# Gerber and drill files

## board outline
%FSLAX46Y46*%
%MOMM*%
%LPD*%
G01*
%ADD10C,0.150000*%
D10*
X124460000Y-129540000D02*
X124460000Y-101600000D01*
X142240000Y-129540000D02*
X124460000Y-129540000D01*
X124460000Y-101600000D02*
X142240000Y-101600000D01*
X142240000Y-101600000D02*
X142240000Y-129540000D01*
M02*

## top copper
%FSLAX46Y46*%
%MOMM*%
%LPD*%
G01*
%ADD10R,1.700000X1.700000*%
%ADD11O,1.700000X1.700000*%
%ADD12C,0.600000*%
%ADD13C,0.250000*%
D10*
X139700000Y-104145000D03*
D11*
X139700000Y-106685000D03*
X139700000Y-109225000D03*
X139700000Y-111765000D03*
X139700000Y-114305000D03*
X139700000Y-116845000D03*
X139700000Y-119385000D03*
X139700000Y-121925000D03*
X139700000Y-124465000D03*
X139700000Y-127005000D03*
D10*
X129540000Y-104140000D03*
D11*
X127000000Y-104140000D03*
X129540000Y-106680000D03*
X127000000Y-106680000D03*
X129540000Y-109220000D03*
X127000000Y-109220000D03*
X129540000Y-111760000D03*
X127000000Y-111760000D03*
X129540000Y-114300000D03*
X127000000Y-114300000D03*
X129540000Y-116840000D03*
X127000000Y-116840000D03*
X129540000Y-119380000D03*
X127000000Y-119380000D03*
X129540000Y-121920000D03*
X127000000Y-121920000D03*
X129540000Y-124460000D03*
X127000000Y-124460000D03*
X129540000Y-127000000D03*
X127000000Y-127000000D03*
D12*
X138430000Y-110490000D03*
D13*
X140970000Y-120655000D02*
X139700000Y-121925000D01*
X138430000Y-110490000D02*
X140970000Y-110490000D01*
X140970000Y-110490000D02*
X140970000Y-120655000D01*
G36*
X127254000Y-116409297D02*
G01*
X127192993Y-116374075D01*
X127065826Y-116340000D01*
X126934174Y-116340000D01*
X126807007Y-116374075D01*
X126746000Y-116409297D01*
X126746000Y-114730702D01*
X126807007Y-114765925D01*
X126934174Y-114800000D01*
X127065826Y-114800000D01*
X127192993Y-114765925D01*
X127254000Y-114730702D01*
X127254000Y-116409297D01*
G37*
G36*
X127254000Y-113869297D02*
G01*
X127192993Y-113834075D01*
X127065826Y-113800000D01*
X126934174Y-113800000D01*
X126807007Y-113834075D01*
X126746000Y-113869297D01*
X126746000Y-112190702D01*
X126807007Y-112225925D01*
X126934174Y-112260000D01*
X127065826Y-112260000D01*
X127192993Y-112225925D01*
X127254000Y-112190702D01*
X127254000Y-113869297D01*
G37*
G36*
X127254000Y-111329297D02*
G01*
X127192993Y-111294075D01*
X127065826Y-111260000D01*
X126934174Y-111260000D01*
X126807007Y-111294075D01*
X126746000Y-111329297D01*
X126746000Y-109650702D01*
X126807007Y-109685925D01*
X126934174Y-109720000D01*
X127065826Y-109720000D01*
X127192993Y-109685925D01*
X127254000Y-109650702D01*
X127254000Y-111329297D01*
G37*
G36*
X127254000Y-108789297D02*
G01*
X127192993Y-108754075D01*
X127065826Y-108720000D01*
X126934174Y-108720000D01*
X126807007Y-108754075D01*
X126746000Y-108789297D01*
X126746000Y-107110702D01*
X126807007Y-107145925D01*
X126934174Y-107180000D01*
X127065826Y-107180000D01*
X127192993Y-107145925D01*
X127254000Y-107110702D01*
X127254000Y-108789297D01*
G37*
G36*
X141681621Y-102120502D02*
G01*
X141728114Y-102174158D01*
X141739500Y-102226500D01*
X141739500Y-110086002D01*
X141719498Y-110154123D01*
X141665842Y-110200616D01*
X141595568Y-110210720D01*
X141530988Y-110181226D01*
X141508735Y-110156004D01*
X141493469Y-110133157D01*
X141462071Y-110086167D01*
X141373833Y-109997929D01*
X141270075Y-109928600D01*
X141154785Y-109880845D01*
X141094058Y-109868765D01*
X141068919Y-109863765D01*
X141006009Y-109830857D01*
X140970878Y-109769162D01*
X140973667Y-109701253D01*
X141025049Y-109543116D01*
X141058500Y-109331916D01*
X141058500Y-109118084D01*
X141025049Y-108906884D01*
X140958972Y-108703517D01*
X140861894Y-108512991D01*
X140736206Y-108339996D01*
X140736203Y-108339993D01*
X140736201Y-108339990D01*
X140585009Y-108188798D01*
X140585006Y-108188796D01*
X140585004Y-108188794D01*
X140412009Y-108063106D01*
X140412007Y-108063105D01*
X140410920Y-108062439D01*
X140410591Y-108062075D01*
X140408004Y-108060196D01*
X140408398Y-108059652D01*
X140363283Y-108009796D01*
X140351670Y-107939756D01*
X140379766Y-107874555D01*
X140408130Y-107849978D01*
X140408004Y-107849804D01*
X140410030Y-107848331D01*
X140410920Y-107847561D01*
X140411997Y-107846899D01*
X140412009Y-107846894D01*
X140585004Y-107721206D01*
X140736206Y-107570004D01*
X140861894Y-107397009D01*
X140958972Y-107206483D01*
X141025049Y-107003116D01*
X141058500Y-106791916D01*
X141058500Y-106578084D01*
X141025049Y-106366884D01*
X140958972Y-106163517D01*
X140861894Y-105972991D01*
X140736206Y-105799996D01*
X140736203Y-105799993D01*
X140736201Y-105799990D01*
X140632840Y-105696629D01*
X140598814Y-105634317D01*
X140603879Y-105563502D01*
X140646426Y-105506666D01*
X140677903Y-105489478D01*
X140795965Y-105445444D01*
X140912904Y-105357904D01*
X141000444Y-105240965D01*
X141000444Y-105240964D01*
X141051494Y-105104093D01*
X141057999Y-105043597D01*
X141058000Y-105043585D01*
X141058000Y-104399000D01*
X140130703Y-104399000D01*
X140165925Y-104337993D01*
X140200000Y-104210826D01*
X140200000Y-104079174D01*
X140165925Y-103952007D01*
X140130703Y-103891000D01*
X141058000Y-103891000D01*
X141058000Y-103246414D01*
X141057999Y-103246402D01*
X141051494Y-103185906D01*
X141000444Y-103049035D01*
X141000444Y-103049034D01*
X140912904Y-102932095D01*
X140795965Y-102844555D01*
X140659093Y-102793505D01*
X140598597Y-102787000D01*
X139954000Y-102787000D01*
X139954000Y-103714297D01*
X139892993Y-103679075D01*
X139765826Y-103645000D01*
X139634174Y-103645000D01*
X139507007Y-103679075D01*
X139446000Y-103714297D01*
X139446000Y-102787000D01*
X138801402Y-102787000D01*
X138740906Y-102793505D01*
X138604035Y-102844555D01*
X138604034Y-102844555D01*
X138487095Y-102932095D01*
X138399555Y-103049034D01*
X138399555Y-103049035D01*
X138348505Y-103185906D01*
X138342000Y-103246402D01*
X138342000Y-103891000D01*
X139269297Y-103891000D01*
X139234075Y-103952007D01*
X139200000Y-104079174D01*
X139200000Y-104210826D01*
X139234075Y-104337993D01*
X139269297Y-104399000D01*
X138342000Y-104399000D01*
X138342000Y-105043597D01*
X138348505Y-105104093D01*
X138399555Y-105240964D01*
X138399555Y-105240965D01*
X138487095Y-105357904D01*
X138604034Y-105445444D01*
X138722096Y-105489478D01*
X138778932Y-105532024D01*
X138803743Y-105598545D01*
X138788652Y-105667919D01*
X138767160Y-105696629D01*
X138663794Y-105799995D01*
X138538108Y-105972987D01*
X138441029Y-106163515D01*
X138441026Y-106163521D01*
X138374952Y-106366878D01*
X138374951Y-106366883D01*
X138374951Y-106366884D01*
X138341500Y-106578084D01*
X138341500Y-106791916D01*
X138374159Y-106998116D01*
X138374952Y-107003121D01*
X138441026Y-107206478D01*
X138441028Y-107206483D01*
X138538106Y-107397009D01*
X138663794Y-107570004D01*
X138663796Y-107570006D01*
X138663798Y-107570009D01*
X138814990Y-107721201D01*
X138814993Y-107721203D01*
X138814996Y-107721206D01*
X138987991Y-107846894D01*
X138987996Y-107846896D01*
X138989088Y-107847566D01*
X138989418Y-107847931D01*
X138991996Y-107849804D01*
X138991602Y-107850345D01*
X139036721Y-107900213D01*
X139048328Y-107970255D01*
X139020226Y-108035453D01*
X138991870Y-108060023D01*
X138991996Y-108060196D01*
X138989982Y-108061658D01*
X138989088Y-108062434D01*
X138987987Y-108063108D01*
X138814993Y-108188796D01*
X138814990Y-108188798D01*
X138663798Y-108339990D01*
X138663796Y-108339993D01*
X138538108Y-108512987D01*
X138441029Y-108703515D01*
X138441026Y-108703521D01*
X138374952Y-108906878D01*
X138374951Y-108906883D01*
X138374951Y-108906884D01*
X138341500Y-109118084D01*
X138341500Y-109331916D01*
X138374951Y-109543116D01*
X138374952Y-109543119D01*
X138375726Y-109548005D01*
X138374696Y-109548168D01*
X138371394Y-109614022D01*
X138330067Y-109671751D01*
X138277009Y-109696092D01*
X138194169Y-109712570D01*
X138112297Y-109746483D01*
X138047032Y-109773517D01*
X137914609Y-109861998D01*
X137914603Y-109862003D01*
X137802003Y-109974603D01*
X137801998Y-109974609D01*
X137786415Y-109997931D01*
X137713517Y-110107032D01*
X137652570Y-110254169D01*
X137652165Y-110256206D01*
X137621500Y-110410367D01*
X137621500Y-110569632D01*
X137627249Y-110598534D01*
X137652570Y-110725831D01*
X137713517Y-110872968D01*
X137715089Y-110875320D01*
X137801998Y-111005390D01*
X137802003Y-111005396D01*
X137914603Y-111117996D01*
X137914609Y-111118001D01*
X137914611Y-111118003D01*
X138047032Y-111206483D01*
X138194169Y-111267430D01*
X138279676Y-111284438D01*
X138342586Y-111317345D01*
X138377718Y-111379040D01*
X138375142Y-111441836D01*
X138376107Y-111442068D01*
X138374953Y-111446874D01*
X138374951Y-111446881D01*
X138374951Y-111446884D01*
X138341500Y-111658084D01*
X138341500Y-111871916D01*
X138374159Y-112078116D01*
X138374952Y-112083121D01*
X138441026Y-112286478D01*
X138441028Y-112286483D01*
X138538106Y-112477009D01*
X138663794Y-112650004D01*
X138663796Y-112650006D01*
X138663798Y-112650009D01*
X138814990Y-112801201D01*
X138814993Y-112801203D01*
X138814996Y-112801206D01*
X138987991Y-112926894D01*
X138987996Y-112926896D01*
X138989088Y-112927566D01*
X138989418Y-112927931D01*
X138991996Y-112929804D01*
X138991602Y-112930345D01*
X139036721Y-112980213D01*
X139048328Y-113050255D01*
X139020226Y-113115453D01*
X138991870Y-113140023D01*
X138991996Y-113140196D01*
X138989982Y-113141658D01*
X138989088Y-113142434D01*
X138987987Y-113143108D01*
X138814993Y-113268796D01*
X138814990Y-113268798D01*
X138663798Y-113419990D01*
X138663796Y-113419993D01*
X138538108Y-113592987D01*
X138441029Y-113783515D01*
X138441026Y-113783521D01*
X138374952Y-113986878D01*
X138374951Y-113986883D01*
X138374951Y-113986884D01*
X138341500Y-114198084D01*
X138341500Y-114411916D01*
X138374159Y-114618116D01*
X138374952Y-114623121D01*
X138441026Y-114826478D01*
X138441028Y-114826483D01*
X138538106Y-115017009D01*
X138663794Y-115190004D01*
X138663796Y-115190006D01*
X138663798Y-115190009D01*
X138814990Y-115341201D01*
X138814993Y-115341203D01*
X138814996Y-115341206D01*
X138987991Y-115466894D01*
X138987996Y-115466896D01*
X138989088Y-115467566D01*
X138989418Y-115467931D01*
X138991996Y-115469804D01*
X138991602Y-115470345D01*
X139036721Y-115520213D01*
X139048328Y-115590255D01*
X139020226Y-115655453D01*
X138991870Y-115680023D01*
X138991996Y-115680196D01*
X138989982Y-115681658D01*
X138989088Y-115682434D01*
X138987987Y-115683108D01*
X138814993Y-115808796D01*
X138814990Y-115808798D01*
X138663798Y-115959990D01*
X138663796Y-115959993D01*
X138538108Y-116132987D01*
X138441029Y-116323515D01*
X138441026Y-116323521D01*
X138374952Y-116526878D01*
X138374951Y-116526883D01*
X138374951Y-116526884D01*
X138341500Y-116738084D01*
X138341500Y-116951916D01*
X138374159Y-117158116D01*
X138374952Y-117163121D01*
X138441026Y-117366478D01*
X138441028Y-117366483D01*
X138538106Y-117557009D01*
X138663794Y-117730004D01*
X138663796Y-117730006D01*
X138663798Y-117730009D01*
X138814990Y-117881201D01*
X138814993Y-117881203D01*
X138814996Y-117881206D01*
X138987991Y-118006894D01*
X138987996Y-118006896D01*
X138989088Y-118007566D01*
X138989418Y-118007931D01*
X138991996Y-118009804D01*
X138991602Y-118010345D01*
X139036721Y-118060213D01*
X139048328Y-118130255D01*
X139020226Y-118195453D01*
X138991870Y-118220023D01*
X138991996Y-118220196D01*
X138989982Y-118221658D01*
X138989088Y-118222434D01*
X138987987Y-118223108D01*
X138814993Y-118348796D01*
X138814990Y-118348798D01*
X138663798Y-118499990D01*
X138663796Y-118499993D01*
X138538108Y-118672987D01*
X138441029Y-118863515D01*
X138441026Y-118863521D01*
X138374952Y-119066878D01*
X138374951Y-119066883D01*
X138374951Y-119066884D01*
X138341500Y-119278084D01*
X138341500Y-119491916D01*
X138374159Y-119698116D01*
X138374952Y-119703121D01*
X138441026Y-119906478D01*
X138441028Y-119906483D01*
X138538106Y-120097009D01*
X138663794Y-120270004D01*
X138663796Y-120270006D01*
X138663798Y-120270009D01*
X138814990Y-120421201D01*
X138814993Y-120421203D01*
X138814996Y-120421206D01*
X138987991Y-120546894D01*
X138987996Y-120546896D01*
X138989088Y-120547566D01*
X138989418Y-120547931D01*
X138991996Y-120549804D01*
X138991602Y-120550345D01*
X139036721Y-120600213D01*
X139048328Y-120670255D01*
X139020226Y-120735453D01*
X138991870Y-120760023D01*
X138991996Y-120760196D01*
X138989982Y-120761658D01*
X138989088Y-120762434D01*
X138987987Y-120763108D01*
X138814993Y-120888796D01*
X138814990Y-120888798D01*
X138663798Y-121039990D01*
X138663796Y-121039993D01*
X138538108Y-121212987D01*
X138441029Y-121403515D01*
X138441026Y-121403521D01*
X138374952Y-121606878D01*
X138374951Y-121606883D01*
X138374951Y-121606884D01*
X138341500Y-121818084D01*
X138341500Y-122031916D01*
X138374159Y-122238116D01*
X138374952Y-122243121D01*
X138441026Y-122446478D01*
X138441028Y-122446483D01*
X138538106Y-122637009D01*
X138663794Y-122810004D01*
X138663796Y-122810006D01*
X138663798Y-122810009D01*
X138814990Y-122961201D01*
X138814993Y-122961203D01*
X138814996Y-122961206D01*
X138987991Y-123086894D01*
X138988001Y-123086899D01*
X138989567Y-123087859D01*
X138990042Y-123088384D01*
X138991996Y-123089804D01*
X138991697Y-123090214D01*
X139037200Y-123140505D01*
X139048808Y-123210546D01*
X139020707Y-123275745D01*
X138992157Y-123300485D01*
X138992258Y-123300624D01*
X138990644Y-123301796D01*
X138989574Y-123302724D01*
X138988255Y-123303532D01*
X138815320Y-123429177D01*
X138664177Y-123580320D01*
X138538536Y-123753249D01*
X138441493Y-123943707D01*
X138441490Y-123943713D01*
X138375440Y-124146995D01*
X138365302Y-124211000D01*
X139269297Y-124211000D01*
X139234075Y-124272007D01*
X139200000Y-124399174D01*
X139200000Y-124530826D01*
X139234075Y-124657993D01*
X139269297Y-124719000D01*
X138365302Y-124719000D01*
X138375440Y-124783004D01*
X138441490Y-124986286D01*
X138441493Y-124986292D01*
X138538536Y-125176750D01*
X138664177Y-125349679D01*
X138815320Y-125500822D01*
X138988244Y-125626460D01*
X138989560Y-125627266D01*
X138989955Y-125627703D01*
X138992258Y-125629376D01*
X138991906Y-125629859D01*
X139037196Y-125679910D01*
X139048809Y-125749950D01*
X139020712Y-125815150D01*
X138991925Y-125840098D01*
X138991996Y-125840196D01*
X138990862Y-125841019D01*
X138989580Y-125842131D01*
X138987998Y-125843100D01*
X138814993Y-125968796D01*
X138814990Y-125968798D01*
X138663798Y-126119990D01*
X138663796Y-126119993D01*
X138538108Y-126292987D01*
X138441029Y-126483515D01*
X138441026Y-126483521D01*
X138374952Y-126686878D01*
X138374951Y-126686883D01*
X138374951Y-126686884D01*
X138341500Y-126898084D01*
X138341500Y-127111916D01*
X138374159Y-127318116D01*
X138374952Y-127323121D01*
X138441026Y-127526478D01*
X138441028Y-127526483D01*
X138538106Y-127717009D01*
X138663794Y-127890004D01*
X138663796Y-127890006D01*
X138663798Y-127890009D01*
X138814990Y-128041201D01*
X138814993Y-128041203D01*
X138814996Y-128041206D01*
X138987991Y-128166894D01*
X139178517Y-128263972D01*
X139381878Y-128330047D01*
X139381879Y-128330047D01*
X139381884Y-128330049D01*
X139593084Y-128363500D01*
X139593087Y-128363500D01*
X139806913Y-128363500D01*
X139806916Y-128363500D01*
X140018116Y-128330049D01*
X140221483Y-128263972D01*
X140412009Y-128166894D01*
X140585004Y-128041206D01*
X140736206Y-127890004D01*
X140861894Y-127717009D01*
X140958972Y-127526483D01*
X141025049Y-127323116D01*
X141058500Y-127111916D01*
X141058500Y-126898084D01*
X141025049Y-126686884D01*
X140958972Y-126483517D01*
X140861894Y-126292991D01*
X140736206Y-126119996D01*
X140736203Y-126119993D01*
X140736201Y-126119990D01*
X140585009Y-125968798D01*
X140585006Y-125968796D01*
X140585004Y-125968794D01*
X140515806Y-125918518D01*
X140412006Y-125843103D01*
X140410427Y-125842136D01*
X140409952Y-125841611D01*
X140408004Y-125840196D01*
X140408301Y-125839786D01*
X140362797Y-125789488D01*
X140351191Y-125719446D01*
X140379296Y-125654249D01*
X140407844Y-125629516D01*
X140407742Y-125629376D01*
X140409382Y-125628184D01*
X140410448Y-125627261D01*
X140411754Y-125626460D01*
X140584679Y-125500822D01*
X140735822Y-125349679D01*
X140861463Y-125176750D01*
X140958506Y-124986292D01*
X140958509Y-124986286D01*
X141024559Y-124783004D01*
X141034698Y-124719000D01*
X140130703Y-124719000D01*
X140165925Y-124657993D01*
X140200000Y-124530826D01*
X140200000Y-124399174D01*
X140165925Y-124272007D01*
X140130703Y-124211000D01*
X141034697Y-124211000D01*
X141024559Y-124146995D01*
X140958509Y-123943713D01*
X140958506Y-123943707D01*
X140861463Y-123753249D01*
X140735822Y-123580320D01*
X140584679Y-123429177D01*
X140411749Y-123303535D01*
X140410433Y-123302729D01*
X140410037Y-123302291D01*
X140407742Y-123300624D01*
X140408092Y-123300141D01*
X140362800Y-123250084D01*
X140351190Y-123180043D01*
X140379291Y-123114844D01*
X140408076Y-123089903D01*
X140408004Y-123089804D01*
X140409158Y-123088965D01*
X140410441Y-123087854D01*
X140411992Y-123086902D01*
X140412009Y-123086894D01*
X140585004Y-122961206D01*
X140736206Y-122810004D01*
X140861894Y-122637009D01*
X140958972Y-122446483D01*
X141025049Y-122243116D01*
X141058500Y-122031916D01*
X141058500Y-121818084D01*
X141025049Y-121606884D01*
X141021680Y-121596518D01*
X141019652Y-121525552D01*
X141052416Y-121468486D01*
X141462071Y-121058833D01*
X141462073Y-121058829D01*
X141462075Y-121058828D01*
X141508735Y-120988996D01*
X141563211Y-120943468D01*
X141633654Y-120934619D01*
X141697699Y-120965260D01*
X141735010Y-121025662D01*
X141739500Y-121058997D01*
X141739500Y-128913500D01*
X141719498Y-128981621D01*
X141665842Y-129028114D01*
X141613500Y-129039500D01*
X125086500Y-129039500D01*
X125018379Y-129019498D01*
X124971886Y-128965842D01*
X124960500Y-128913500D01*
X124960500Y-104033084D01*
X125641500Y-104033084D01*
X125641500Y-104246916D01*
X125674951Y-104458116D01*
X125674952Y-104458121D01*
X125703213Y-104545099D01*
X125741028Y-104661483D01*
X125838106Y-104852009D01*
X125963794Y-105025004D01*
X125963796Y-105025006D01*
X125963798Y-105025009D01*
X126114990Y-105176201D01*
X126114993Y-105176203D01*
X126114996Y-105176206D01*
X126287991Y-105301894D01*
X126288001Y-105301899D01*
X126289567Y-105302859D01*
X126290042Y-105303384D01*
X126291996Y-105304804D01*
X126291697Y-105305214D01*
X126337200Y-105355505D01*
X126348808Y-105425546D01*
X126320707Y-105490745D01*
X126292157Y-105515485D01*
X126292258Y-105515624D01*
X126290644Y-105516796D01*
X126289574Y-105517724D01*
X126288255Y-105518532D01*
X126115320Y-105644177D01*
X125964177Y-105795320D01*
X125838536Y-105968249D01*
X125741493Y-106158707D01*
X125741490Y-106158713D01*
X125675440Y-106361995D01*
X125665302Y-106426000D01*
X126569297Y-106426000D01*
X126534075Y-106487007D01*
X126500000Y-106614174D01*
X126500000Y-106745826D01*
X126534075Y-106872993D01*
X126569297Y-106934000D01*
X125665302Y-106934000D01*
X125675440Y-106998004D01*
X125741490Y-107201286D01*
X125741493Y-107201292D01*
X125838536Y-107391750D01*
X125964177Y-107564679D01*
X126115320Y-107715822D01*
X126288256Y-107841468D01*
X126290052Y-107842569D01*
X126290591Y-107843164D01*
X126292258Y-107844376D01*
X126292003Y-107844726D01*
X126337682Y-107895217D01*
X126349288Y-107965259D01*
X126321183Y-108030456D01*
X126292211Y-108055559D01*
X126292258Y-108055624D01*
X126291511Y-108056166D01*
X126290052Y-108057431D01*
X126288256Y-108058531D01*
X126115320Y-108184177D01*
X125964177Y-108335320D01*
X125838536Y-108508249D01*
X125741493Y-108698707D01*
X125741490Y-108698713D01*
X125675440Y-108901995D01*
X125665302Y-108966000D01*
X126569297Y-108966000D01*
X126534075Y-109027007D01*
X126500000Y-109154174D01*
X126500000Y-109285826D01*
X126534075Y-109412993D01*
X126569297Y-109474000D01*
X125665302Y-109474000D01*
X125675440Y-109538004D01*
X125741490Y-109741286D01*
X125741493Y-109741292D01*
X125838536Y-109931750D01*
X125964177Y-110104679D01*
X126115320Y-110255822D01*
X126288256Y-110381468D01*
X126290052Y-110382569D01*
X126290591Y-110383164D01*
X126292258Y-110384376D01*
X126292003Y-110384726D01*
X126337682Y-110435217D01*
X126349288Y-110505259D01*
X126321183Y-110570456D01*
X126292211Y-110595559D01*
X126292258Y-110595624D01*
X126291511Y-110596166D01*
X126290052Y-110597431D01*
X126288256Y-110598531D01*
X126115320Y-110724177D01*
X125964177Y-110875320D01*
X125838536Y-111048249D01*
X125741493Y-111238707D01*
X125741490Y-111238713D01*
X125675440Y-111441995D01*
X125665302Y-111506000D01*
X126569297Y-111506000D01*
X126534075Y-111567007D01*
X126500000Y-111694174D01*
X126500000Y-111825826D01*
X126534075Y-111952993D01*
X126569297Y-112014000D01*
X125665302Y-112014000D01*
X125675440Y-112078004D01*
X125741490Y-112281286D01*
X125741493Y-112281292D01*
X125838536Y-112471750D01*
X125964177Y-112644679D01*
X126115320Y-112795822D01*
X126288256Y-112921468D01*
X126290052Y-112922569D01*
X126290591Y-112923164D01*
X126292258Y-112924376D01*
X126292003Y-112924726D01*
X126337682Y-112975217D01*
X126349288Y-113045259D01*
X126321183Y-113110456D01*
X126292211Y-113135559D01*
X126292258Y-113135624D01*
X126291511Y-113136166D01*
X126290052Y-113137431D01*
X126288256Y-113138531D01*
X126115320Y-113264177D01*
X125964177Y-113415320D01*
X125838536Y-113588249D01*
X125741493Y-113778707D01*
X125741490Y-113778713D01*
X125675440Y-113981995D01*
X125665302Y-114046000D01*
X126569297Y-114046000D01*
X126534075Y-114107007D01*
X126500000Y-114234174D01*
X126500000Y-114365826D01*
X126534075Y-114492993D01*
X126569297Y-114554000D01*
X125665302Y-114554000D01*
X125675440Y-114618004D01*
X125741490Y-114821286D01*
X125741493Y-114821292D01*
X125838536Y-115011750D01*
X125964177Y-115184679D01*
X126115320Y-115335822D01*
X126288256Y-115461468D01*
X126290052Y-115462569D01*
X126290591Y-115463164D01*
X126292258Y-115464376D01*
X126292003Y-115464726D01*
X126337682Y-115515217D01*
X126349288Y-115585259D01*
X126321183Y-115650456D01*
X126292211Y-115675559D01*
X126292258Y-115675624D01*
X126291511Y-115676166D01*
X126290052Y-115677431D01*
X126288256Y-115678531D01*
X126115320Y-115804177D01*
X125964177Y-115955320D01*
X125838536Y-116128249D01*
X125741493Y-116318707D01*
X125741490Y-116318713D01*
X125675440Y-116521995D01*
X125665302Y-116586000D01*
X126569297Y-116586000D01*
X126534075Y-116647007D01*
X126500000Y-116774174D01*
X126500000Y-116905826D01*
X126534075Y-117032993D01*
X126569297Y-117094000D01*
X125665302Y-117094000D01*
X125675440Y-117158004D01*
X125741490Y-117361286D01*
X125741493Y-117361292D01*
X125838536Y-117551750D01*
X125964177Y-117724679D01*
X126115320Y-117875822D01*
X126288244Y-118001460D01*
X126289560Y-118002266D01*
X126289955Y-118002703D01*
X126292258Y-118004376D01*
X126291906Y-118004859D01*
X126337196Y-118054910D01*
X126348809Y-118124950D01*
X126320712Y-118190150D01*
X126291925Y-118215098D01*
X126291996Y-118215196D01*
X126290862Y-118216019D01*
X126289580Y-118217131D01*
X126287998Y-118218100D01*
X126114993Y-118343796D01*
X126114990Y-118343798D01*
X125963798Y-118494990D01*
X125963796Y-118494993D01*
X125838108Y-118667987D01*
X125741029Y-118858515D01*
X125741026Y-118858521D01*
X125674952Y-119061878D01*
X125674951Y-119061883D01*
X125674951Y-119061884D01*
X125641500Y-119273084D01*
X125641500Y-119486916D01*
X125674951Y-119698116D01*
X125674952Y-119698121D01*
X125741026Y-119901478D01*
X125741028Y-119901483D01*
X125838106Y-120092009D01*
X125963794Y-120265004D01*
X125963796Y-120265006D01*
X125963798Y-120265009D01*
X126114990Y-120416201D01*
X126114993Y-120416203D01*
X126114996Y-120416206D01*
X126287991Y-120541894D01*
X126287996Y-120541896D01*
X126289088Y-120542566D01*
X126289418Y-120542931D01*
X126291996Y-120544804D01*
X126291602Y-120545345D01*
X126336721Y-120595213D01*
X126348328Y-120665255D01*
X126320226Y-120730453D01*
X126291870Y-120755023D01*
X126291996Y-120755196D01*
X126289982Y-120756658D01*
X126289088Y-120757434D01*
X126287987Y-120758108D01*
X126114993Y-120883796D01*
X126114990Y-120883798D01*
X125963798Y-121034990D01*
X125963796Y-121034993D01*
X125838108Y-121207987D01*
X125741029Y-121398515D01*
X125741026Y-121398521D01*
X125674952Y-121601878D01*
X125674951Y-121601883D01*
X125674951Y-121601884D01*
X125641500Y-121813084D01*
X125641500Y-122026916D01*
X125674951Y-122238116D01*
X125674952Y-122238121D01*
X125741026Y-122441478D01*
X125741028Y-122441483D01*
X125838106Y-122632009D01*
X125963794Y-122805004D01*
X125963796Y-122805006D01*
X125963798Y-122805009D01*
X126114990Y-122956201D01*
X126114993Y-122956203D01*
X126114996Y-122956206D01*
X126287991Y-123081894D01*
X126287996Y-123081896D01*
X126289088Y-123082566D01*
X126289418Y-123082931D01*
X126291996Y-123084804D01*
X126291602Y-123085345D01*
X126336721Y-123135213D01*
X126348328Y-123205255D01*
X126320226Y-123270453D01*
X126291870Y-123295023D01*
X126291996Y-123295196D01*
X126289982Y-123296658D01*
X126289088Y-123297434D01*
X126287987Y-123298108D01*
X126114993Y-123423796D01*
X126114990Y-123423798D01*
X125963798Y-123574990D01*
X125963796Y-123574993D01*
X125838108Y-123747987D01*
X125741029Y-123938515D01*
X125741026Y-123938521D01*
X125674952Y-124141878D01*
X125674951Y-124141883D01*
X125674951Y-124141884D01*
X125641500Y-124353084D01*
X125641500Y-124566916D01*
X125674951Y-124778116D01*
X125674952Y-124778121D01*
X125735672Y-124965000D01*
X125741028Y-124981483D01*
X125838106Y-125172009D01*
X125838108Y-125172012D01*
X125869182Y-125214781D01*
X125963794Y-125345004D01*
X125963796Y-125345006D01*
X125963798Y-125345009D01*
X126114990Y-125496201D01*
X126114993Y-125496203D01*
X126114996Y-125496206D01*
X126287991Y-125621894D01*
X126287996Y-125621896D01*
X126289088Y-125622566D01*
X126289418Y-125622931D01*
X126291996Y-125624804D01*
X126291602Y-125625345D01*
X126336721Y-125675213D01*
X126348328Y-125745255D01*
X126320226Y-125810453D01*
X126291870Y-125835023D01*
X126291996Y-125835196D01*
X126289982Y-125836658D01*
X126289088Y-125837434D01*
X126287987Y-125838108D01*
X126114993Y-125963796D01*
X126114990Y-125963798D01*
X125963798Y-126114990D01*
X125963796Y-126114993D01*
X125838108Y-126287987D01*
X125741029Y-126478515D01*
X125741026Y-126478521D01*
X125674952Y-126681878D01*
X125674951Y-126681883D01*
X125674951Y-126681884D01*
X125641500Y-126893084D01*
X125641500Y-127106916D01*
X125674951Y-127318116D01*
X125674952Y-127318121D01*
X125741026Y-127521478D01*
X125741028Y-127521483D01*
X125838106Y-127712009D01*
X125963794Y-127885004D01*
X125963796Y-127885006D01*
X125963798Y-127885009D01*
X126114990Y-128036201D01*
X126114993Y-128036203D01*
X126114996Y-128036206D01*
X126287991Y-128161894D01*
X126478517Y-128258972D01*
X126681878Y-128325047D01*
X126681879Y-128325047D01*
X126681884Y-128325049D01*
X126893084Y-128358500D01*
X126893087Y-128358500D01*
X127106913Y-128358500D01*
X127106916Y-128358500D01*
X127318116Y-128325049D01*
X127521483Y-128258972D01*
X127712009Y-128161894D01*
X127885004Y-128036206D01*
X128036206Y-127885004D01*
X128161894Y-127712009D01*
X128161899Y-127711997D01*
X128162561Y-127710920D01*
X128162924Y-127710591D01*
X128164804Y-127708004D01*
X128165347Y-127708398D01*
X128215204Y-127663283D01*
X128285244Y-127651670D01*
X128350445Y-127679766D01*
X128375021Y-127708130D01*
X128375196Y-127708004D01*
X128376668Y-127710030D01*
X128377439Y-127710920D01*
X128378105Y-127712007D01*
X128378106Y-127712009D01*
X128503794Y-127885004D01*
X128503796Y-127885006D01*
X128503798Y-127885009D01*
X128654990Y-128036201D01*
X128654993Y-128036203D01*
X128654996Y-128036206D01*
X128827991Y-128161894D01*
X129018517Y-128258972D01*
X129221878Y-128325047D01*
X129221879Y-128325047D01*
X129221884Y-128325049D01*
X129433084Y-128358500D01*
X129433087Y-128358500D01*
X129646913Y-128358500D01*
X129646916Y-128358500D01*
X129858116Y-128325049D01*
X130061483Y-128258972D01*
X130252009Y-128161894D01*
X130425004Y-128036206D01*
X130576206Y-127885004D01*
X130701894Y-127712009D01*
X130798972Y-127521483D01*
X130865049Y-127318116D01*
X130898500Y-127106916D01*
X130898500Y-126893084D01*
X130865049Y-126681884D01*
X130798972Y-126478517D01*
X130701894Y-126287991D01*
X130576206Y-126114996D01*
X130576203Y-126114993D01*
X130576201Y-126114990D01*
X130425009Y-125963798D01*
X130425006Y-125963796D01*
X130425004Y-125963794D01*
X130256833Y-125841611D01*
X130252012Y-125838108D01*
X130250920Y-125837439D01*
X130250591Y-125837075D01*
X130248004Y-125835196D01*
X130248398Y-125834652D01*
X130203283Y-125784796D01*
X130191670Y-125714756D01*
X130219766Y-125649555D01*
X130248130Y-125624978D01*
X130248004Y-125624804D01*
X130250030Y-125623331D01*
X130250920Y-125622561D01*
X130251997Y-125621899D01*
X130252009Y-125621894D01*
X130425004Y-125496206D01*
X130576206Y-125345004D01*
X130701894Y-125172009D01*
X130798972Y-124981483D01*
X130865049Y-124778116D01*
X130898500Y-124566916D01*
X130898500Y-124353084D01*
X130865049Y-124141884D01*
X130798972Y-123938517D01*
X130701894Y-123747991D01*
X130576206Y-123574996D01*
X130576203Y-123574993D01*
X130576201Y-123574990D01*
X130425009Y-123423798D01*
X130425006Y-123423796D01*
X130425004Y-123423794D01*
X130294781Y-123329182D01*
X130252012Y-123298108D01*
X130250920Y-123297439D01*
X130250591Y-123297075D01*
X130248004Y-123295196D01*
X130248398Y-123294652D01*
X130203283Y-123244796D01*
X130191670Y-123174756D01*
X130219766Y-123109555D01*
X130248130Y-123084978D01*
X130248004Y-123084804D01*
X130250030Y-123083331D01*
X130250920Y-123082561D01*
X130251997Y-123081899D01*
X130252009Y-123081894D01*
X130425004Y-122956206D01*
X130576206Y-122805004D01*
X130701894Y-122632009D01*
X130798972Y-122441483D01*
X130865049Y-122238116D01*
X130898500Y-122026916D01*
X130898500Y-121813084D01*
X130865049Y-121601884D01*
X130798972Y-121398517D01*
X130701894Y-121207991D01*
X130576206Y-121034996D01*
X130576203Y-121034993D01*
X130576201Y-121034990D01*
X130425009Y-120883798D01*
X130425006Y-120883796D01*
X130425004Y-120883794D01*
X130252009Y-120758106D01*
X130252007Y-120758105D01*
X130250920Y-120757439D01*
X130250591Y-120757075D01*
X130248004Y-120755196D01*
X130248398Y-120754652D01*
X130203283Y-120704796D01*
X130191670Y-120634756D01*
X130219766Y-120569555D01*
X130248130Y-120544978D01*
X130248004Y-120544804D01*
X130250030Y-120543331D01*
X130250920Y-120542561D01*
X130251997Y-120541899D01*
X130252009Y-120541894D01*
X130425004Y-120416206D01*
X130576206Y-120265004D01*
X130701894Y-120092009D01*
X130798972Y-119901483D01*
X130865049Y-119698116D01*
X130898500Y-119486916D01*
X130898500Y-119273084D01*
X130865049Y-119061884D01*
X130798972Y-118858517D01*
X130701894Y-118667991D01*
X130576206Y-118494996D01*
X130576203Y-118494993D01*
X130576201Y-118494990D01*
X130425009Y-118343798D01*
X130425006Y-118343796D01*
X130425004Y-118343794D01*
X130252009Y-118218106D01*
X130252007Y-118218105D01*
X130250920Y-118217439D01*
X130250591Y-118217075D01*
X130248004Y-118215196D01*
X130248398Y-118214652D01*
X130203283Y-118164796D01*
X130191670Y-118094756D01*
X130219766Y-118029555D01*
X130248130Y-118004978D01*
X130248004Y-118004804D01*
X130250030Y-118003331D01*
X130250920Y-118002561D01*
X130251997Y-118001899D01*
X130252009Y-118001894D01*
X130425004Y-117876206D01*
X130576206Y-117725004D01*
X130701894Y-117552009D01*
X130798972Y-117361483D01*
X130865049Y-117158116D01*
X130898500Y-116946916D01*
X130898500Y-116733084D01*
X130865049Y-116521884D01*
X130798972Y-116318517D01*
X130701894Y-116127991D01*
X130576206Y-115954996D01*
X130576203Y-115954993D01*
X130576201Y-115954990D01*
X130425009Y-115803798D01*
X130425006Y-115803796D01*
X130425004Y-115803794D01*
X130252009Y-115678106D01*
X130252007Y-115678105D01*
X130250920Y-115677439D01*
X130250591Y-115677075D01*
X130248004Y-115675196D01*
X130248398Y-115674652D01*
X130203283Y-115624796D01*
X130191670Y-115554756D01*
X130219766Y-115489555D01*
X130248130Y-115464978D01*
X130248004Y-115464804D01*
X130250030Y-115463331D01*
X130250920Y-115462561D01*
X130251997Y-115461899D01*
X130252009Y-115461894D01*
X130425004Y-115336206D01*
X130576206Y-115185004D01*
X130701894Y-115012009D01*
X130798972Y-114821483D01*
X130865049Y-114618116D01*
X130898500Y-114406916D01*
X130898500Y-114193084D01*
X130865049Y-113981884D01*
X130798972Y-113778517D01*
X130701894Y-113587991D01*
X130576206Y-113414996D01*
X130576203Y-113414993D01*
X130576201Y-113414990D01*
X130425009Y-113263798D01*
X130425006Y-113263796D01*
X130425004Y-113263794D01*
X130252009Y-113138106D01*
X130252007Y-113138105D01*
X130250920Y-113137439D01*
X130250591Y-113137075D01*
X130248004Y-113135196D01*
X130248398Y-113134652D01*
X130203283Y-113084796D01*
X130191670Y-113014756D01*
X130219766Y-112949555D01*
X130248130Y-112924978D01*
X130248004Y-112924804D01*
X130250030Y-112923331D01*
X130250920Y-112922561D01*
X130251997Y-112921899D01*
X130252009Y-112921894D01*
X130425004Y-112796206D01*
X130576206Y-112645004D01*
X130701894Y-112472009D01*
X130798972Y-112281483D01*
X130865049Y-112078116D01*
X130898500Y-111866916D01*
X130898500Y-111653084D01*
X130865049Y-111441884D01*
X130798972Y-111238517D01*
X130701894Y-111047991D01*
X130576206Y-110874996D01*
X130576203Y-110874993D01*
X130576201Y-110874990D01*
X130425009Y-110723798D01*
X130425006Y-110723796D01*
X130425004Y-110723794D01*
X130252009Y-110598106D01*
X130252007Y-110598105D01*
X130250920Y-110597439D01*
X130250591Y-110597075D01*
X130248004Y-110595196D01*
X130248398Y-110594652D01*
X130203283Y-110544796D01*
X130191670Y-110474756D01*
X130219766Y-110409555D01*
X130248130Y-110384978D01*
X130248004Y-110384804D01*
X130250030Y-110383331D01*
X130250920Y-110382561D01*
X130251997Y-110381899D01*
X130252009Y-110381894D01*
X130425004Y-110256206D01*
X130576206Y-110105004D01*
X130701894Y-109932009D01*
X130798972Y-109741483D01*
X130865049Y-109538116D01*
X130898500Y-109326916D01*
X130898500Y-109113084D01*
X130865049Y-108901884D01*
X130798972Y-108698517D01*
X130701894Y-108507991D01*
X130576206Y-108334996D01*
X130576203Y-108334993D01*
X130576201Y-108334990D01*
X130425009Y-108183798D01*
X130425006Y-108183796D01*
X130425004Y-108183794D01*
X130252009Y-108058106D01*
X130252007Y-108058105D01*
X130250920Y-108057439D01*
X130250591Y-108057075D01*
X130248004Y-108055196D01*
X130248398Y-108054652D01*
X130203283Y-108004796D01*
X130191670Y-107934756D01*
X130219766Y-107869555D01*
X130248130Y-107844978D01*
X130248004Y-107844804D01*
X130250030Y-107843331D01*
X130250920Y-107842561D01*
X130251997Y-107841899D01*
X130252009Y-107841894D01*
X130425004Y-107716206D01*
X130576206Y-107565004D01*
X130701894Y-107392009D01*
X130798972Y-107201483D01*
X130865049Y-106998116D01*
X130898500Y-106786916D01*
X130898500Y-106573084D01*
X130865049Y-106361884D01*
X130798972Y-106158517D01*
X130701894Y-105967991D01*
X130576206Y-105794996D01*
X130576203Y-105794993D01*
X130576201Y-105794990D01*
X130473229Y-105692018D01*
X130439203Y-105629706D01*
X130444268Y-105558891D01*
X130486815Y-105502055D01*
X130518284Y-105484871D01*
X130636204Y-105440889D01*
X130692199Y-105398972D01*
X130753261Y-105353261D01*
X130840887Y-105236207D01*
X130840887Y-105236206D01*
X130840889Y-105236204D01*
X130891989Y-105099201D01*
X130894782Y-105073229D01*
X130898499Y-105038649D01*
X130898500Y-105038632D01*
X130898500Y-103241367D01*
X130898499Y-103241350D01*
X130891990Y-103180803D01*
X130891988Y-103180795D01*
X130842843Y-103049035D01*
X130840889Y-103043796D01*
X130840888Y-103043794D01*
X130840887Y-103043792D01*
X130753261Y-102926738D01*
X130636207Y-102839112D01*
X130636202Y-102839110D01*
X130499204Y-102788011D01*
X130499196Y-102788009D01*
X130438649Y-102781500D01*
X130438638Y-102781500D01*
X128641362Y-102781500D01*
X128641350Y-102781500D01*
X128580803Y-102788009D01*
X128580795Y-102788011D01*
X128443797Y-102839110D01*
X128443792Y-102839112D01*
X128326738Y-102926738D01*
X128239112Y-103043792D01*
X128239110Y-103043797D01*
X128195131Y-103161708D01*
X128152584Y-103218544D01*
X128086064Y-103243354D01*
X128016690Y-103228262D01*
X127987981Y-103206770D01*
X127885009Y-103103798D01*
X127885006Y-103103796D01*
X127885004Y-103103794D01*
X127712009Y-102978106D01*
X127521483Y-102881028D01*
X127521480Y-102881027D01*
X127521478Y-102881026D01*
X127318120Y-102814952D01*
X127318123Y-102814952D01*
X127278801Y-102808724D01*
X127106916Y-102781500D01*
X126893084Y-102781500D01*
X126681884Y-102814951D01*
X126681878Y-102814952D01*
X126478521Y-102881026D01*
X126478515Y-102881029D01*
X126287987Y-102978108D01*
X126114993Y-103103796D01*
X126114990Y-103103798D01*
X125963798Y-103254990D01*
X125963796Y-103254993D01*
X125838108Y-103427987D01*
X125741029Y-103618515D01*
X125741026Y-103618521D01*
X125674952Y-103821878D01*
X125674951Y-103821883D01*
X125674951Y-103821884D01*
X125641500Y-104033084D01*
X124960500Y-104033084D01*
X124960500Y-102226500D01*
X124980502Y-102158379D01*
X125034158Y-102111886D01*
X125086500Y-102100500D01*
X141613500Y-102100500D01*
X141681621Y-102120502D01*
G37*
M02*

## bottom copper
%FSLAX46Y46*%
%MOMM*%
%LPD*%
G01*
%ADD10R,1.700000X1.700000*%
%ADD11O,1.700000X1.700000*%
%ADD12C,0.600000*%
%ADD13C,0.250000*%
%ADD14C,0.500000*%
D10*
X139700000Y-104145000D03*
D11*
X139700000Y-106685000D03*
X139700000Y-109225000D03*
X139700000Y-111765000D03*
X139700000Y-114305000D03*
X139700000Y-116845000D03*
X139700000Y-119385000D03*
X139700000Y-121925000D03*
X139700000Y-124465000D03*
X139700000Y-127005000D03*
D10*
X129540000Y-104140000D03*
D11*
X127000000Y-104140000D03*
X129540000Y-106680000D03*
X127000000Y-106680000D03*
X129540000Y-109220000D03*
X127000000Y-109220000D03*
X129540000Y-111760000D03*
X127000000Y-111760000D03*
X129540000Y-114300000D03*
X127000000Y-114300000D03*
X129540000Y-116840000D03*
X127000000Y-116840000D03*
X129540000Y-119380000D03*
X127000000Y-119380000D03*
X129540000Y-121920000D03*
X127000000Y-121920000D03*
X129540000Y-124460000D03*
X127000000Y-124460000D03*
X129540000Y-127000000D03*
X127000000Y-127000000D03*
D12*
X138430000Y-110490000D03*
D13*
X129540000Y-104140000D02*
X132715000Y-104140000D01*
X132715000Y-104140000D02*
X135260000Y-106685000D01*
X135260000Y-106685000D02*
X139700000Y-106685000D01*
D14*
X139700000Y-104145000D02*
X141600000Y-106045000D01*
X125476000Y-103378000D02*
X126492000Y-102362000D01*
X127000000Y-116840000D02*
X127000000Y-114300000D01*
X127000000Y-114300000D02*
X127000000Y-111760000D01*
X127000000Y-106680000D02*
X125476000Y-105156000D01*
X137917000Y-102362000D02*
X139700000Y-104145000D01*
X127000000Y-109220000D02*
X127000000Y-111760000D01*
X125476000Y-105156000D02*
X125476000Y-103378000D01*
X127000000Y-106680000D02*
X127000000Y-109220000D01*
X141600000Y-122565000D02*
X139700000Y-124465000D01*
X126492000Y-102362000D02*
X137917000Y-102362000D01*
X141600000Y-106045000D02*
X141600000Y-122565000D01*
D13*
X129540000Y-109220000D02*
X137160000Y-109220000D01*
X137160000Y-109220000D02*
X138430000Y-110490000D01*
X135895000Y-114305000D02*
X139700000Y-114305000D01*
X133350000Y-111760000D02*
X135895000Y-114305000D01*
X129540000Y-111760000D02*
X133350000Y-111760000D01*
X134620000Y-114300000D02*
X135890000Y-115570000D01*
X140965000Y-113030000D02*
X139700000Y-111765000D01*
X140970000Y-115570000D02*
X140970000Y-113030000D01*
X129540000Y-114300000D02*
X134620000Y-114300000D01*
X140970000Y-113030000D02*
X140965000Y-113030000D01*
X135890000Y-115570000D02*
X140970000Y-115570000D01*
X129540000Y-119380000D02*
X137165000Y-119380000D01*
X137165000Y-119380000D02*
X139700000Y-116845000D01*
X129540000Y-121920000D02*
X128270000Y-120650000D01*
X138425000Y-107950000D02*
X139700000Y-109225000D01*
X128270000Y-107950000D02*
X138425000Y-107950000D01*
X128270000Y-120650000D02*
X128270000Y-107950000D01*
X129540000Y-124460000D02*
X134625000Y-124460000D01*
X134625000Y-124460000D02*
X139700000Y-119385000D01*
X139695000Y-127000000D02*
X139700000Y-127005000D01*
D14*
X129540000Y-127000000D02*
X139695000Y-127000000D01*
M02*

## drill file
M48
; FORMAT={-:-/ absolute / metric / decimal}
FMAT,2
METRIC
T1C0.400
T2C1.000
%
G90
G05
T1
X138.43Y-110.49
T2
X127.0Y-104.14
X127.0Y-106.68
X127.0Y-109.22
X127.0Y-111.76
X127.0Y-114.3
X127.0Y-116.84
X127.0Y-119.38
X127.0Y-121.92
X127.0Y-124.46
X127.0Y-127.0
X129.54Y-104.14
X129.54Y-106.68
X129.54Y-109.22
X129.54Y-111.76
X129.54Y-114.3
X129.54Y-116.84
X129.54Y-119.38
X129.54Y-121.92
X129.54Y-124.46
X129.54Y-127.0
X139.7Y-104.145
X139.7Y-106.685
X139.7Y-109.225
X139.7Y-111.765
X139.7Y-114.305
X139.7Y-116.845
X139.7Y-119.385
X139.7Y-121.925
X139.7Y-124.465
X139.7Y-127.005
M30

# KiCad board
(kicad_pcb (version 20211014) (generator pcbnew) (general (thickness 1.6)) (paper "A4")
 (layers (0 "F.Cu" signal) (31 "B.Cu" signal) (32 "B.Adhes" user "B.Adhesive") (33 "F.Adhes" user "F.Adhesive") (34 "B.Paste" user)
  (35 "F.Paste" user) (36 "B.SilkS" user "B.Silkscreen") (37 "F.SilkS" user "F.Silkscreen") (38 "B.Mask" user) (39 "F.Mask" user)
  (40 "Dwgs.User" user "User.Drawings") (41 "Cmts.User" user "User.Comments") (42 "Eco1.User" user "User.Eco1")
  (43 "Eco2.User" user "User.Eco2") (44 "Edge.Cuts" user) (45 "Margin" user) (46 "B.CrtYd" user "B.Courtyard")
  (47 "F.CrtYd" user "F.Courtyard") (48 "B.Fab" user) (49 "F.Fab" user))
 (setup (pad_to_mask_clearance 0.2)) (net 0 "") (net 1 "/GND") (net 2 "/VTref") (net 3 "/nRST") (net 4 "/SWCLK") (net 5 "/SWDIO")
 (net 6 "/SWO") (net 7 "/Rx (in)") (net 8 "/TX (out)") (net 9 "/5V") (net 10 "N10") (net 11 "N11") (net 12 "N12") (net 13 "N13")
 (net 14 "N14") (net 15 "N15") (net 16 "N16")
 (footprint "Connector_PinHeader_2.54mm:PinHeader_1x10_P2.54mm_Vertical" (layer "F.Cu") (at 139.7 104.145)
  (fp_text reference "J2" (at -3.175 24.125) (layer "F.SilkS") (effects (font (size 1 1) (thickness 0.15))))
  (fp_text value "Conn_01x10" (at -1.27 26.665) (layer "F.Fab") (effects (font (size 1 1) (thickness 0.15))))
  (pad "1" thru_hole rect (at 0 0) (size 1.7 1.7) (drill 1) (layers *.Cu *.Mask) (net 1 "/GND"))
  (pad "2" thru_hole oval (at 0 2.54) (size 1.7 1.7) (drill 1) (layers *.Cu *.Mask) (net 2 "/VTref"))
  (pad "3" thru_hole oval (at 0 5.08) (size 1.7 1.7) (drill 1) (layers *.Cu *.Mask) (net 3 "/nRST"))
  (pad "4" thru_hole oval (at 0 7.62) (size 1.7 1.7) (drill 1) (layers *.Cu *.Mask) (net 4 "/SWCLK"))
  (pad "5" thru_hole oval (at 0 10.16) (size 1.7 1.7) (drill 1) (layers *.Cu *.Mask) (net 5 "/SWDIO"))
  (pad "6" thru_hole oval (at 0 12.7) (size 1.7 1.7) (drill 1) (layers *.Cu *.Mask) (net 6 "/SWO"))
  (pad "7" thru_hole oval (at 0 15.24) (size 1.7 1.7) (drill 1) (layers *.Cu *.Mask) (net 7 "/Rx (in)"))
  (pad "8" thru_hole oval (at 0 17.78) (size 1.7 1.7) (drill 1) (layers *.Cu *.Mask) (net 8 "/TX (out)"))
  (pad "9" thru_hole oval (at 0 20.32) (size 1.7 1.7) (drill 1) (layers *.Cu *.Mask) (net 1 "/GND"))
  (pad "10" thru_hole oval (at 0 22.86) (size 1.7 1.7) (drill 1) (layers *.Cu *.Mask) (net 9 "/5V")))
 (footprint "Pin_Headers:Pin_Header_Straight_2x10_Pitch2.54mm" (layer "B.Cu") (at 129.54 104.14 180)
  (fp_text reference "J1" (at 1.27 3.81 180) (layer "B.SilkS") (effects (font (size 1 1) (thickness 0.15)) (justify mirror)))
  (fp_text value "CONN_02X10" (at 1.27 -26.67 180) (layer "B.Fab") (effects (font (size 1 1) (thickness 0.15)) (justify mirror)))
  (pad "1" thru_hole rect locked (at 0 0 180) (size 1.7 1.7) (drill 1) (layers *.Cu *.Mask) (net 2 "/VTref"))
  (pad "2" thru_hole oval locked (at 2.54 0 180) (size 1.7 1.7) (drill 1) (layers *.Cu *.Mask) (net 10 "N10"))
  (pad "3" thru_hole oval locked (at 0 -2.54 180) (size 1.7 1.7) (drill 1) (layers *.Cu *.Mask) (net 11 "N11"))
  (pad "4" thru_hole oval locked (at 2.54 -2.54 180) (size 1.7 1.7) (drill 1) (layers *.Cu *.Mask) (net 1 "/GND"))
  (pad "5" thru_hole oval locked (at 0 -5.08 180) (size 1.7 1.7) (drill 1) (layers *.Cu *.Mask) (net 8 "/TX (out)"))
  (pad "6" thru_hole oval locked (at 2.54 -5.08 180) (size 1.7 1.7) (drill 1) (layers *.Cu *.Mask) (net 1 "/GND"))
  (pad "7" thru_hole oval locked (at 0 -7.62 180) (size 1.7 1.7) (drill 1) (layers *.Cu *.Mask) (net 5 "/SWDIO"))
  (pad "8" thru_hole oval locked (at 2.54 -7.62 180) (size 1.7 1.7) (drill 1) (layers *.Cu *.Mask) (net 1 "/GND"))
  (pad "9" thru_hole oval locked (at 0 -10.16 180) (size 1.7 1.7) (drill 1) (layers *.Cu *.Mask) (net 4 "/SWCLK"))
  (pad "10" thru_hole oval locked (at 2.54 -10.16 180) (size 1.7 1.7) (drill 1) (layers *.Cu *.Mask) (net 1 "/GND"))
  (pad "11" thru_hole oval locked (at 0 -12.7 180) (size 1.7 1.7) (drill 1) (layers *.Cu *.Mask) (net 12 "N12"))
  (pad "12" thru_hole oval locked (at 2.54 -12.7 180) (size 1.7 1.7) (drill 1) (layers *.Cu *.Mask) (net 1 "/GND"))
  (pad "13" thru_hole oval locked (at 0 -15.24 180) (size 1.7 1.7) (drill 1) (layers *.Cu *.Mask) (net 6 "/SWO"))
  (pad "14" thru_hole oval locked (at 2.54 -15.24 180) (size 1.7 1.7) (drill 1) (layers *.Cu *.Mask) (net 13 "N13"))
  (pad "15" thru_hole oval locked (at 0 -17.78 180) (size 1.7 1.7) (drill 1) (layers *.Cu *.Mask) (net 3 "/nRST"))
  (pad "16" thru_hole oval locked (at 2.54 -17.78 180) (size 1.7 1.7) (drill 1) (layers *.Cu *.Mask) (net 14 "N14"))
  (pad "17" thru_hole oval locked (at 0 -20.32 180) (size 1.7 1.7) (drill 1) (layers *.Cu *.Mask) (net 7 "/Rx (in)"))
  (pad "18" thru_hole oval locked (at 2.54 -20.32 180) (size 1.7 1.7) (drill 1) (layers *.Cu *.Mask) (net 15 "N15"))
  (pad "19" thru_hole oval locked (at 0 -22.86 180) (size 1.7 1.7) (drill 1) (layers *.Cu *.Mask) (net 9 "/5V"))
  (pad "20" thru_hole oval locked (at 2.54 -22.86 180) (size 1.7 1.7) (drill 1) (layers *.Cu *.Mask) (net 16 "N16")))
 (gr_line (start 124.46 129.54) (end 124.46 101.6) (layer "Edge.Cuts") (width 0.15))
 (gr_line (start 142.24 129.54) (end 124.46 129.54) (layer "Edge.Cuts") (width 0.15))
 (gr_line (start 124.46 101.6) (end 142.24 101.6) (layer "Edge.Cuts") (width 0.15))
 (gr_line (start 142.24 101.6) (end 142.24 129.54) (layer "Edge.Cuts") (width 0.15))
 (segment (start 129.54 104.14) (end 132.715 104.14) (width 0.25) (layer "B.Cu") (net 2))
 (segment (start 132.715 104.14) (end 135.26 106.685) (width 0.25) (layer "B.Cu") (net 2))
 (segment (start 135.26 106.685) (end 139.7 106.685) (width 0.25) (layer "B.Cu") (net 2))
 (segment (start 139.7 104.145) (end 141.6 106.045) (width 0.5) (layer "B.Cu") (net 1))
 (segment (start 125.476 103.378) (end 126.492 102.362) (width 0.5) (layer "B.Cu") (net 1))
 (segment (start 127 116.84) (end 127 114.3) (width 0.5) (layer "B.Cu") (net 1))
 (segment (start 127 114.3) (end 127 111.76) (width 0.5) (layer "B.Cu") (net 1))
 (segment (start 127 106.68) (end 125.476 105.156) (width 0.5) (layer "B.Cu") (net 1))
 (segment (start 137.917 102.362) (end 139.7 104.145) (width 0.5) (layer "B.Cu") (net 1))
 (segment (start 127 109.22) (end 127 111.76) (width 0.5) (layer "B.Cu") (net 1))
 (segment (start 125.476 105.156) (end 125.476 103.378) (width 0.5) (layer "B.Cu") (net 1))
 (segment (start 127 106.68) (end 127 109.22) (width 0.5) (layer "B.Cu") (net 1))
 (segment (start 141.6 122.565) (end 139.7 124.465) (width 0.5) (layer "B.Cu") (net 1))
 (segment (start 126.492 102.362) (end 137.917 102.362) (width 0.5) (layer "B.Cu") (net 1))
 (segment (start 141.6 106.045) (end 141.6 122.565) (width 0.5) (layer "B.Cu") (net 1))
 (segment (start 140.97 120.655) (end 139.7 121.925) (width 0.25) (layer "F.Cu") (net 8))
 (segment (start 138.43 110.49) (end 140.97 110.49) (width 0.25) (layer "F.Cu") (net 8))
 (segment (start 140.97 110.49) (end 140.97 120.655) (width 0.25) (layer "F.Cu") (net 8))
 (via (at 138.43 110.49) (size 0.6) (drill 0.4) (layers "F.Cu" "B.Cu") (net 8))
 (segment (start 129.54 109.22) (end 137.16 109.22) (width 0.25) (layer "B.Cu") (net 8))
 (segment (start 137.16 109.22) (end 138.43 110.49) (width 0.25) (layer "B.Cu") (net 8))
 (segment (start 135.895 114.305) (end 139.7 114.305) (width 0.25) (layer "B.Cu") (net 5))
 (segment (start 133.35 111.76) (end 135.895 114.305) (width 0.25) (layer "B.Cu") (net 5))
 (segment (start 129.54 111.76) (end 133.35 111.76) (width 0.25) (layer "B.Cu") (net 5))
 (segment (start 134.62 114.3) (end 135.89 115.57) (width 0.25) (layer "B.Cu") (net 4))
 (segment (start 140.965 113.03) (end 139.7 111.765) (width 0.25) (layer "B.Cu") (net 4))
 (segment (start 140.97 115.57) (end 140.97 113.03) (width 0.25) (layer "B.Cu") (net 4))
 (segment (start 129.54 114.3) (end 134.62 114.3) (width 0.25) (layer "B.Cu") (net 4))
 (segment (start 140.97 113.03) (end 140.965 113.03) (width 0.25) (layer "B.Cu") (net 4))
 (segment (start 135.89 115.57) (end 140.97 115.57) (width 0.25) (layer "B.Cu") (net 4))
 (segment (start 129.54 119.38) (end 137.165 119.38) (width 0.25) (layer "B.Cu") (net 6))
 (segment (start 137.165 119.38) (end 139.7 116.845) (width 0.25) (layer "B.Cu") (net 6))
 (segment (start 129.54 121.92) (end 128.27 120.65) (width 0.25) (layer "B.Cu") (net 3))
 (segment (start 138.425 107.95) (end 139.7 109.225) (width 0.25) (layer "B.Cu") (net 3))
 (segment (start 128.27 107.95) (end 138.425 107.95) (width 0.25) (layer "B.Cu") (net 3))
 (segment (start 128.27 120.65) (end 128.27 107.95) (width 0.25) (layer "B.Cu") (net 3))
 (segment (start 129.54 124.46) (end 134.625 124.46) (width 0.25) (layer "B.Cu") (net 7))
 (segment (start 134.625 124.46) (end 139.7 119.385) (width 0.25) (layer "B.Cu") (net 7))
 (segment (start 139.695 127) (end 139.7 127.005) (width 0.25) (layer "B.Cu") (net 9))
 (segment (start 129.54 127) (end 139.695 127) (width 0.5) (layer "B.Cu") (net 9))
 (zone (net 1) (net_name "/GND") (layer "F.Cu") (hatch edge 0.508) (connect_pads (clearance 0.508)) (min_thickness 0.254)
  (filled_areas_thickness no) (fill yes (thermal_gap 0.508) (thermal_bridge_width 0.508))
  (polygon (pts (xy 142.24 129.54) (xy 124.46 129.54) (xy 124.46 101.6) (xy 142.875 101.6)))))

